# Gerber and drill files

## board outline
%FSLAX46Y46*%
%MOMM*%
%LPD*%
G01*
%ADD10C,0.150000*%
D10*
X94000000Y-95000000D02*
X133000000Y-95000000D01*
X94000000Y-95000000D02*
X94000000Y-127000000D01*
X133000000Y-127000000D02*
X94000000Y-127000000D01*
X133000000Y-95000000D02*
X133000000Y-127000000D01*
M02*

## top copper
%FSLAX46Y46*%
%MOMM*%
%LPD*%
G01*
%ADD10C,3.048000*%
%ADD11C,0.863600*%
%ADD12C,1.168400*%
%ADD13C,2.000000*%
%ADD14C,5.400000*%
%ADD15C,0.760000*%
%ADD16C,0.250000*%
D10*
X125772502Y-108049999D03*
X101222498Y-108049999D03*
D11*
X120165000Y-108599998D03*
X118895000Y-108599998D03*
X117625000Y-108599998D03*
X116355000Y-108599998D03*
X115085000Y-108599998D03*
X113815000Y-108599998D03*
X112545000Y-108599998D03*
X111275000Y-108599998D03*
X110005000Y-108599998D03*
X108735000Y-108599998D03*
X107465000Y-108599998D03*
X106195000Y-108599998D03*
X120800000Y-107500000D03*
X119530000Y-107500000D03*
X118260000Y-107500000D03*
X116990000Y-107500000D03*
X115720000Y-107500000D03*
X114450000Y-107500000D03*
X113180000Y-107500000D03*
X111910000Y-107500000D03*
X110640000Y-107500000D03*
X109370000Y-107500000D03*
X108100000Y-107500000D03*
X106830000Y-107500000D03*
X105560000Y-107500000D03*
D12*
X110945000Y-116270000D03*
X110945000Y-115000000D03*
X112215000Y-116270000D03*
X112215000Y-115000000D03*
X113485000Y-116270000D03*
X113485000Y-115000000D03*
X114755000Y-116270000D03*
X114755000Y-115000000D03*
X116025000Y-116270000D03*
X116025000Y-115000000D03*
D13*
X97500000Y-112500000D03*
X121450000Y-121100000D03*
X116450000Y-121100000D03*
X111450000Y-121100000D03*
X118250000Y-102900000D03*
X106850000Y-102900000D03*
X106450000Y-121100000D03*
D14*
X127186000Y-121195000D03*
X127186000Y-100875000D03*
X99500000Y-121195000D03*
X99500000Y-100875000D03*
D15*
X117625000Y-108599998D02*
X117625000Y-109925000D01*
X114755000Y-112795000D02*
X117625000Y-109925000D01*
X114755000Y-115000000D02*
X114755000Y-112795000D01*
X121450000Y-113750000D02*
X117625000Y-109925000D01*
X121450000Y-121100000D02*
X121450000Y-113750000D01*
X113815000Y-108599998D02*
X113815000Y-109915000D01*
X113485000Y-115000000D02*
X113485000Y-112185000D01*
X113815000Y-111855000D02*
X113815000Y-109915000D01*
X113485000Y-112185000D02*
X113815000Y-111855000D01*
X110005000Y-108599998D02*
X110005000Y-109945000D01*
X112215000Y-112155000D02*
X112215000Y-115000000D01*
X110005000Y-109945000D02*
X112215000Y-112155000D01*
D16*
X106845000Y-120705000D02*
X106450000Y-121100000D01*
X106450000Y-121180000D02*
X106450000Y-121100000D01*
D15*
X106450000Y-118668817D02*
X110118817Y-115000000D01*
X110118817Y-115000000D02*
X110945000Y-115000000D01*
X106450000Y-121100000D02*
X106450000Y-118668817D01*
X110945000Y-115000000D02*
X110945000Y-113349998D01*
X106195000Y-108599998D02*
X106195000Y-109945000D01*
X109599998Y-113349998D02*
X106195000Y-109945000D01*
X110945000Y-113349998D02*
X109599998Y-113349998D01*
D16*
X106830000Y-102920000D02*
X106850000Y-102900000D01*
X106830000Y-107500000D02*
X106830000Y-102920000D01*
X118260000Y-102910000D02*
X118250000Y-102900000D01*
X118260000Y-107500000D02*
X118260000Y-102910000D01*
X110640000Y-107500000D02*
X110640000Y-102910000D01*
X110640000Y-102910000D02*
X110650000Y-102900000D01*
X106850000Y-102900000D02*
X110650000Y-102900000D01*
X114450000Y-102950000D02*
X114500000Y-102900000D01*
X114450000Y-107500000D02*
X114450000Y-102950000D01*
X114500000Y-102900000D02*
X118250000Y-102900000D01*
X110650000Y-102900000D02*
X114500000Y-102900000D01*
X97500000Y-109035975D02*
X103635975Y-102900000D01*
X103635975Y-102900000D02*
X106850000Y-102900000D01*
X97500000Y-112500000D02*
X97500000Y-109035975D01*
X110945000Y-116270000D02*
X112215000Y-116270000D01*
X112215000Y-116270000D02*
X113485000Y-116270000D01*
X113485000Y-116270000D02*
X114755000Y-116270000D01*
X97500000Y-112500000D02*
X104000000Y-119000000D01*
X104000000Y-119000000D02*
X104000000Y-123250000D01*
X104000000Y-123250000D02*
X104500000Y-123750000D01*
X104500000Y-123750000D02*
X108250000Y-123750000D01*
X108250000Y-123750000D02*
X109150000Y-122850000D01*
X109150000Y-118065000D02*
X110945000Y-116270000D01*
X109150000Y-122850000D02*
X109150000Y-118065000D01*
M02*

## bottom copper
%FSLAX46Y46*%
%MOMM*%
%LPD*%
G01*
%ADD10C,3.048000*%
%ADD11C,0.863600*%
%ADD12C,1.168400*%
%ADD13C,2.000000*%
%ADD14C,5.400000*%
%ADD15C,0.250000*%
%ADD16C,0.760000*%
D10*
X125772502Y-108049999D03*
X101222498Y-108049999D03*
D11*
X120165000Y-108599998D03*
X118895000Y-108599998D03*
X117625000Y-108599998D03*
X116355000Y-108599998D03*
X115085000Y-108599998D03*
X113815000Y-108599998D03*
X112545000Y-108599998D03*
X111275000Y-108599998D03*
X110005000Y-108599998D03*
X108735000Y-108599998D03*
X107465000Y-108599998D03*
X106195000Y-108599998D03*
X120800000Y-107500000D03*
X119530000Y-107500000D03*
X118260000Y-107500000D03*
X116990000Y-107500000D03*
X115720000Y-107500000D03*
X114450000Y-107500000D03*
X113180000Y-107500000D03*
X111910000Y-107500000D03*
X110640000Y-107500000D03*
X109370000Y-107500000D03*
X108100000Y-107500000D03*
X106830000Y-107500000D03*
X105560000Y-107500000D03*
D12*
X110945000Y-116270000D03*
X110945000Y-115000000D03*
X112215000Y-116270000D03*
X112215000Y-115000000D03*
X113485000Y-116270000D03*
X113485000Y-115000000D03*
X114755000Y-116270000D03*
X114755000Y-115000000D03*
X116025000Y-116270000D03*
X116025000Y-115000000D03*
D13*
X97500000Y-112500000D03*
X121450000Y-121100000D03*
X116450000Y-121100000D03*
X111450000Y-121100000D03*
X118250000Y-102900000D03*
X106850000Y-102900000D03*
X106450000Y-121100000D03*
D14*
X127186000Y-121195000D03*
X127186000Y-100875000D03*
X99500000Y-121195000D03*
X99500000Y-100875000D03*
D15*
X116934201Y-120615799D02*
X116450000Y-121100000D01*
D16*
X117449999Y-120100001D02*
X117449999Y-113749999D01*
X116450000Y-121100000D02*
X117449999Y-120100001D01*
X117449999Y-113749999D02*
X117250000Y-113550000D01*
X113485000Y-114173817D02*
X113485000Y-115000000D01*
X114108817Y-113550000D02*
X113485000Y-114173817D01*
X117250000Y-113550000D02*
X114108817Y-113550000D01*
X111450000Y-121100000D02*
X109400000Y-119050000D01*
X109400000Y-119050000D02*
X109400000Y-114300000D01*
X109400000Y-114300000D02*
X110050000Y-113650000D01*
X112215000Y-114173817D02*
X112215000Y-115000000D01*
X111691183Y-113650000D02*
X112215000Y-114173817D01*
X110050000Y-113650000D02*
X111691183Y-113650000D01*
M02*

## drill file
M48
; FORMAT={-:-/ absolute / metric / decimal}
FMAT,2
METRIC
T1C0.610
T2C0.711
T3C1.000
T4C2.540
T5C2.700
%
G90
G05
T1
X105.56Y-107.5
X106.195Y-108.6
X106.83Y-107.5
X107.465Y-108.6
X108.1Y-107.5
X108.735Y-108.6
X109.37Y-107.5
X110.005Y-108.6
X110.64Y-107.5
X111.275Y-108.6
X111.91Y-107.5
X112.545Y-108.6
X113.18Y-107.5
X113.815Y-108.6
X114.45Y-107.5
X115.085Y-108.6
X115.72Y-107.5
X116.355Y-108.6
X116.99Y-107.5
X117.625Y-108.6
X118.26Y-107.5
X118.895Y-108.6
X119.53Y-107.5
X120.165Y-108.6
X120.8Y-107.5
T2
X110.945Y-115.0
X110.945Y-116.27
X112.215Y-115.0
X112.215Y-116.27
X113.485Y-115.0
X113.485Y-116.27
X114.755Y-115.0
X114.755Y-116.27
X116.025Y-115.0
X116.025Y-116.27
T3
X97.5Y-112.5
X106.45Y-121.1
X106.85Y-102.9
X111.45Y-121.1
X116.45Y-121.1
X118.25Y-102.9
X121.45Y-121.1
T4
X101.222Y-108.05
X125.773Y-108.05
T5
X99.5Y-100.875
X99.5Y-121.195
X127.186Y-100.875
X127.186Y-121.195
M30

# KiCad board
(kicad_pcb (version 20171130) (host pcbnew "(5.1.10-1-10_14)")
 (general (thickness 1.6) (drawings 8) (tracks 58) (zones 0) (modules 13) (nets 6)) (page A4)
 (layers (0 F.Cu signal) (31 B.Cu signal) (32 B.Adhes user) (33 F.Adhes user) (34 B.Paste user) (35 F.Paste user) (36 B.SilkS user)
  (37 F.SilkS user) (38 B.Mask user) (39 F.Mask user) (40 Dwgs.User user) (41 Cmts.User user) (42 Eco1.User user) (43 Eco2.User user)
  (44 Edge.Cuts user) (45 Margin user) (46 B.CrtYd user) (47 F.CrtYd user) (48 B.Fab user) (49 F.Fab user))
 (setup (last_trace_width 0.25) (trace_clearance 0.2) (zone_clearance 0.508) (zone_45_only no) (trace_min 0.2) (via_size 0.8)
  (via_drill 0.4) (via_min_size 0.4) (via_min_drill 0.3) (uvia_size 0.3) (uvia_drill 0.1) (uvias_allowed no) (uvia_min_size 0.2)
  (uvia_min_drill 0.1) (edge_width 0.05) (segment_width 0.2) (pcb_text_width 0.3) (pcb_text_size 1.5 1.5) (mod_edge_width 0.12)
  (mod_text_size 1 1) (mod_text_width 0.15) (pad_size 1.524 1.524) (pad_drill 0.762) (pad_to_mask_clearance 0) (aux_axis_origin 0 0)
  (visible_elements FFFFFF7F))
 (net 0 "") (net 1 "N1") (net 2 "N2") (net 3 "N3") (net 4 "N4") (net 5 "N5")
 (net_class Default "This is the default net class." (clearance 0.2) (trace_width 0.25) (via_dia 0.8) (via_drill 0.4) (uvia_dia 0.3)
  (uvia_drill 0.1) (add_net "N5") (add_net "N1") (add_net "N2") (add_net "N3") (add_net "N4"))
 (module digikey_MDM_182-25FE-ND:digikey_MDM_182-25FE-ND (layer F.Cu) (at 120.8 107.5)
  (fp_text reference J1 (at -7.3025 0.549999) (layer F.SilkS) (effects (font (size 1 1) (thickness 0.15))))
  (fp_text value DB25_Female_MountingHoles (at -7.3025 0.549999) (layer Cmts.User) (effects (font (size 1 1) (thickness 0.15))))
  (pad 28 thru_hole circle (at 4.972502 0.549999 90) (size 3.048 3.048) (drill 2.54) (layers *.Cu *.Mask))
  (pad 27 thru_hole circle (at -19.577502 0.549999 90) (size 3.048 3.048) (drill 2.54) (layers *.Cu *.Mask))
  (pad 14 thru_hole circle (at -0.635 1.099998) (size 0.8636 0.8636) (drill 0.6096) (layers *.Cu *.Mask))
  (pad 15 thru_hole circle (at -1.905 1.099998) (size 0.8636 0.8636) (drill 0.6096) (layers *.Cu *.Mask))
  (pad 16 thru_hole circle (at -3.175 1.099998) (size 0.8636 0.8636) (drill 0.6096) (layers *.Cu *.Mask) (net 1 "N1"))
  (pad 17 thru_hole circle (at -4.445 1.099998) (size 0.8636 0.8636) (drill 0.6096) (layers *.Cu *.Mask))
  (pad 18 thru_hole circle (at -5.715 1.099998) (size 0.8636 0.8636) (drill 0.6096) (layers *.Cu *.Mask))
  (pad 19 thru_hole circle (at -6.985 1.099998) (size 0.8636 0.8636) (drill 0.6096) (layers *.Cu *.Mask) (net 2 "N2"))
  (pad 20 thru_hole circle (at -8.255 1.099998) (size 0.8636 0.8636) (drill 0.6096) (layers *.Cu *.Mask))
  (pad 21 thru_hole circle (at -9.525 1.099998) (size 0.8636 0.8636) (drill 0.6096) (layers *.Cu *.Mask))
  (pad 22 thru_hole circle (at -10.795 1.099998) (size 0.8636 0.8636) (drill 0.6096) (layers *.Cu *.Mask) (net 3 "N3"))
  (pad 23 thru_hole circle (at -12.065 1.099998) (size 0.8636 0.8636) (drill 0.6096) (layers *.Cu *.Mask))
  (pad 24 thru_hole circle (at -13.335 1.099998) (size 0.8636 0.8636) (drill 0.6096) (layers *.Cu *.Mask))
  (pad 25 thru_hole circle (at -14.605 1.099998) (size 0.8636 0.8636) (drill 0.6096) (layers *.Cu *.Mask) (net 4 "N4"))
  (pad 1 thru_hole circle (at 0 0) (size 0.8636 0.8636) (drill 0.6096) (layers *.Cu *.Mask))
  (pad 2 thru_hole circle (at -1.27 0) (size 0.8636 0.8636) (drill 0.6096) (layers *.Cu *.Mask))
  (pad 3 thru_hole circle (at -2.54 0) (size 0.8636 0.8636) (drill 0.6096) (layers *.Cu *.Mask) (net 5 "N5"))
  (pad 4 thru_hole circle (at -3.81 0) (size 0.8636 0.8636) (drill 0.6096) (layers *.Cu *.Mask))
  (pad 5 thru_hole circle (at -5.08 0) (size 0.8636 0.8636) (drill 0.6096) (layers *.Cu *.Mask))
  (pad 6 thru_hole circle (at -6.35 0) (size 0.8636 0.8636) (drill 0.6096) (layers *.Cu *.Mask) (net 5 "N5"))
  (pad 7 thru_hole circle (at -7.62 0) (size 0.8636 0.8636) (drill 0.6096) (layers *.Cu *.Mask))
  (pad 8 thru_hole circle (at -8.89 0) (size 0.8636 0.8636) (drill 0.6096) (layers *.Cu *.Mask))
  (pad 9 thru_hole circle (at -10.16 0) (size 0.8636 0.8636) (drill 0.6096) (layers *.Cu *.Mask) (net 5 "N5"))
  (pad 10 thru_hole circle (at -11.43 0) (size 0.8636 0.8636) (drill 0.6096) (layers *.Cu *.Mask))
  (pad 11 thru_hole circle (at -12.7 0) (size 0.8636 0.8636) (drill 0.6096) (layers *.Cu *.Mask))
  (pad 12 thru_hole circle (at -13.97 0) (size 0.8636 0.8636) (drill 0.6096) (layers *.Cu *.Mask) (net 5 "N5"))
  (pad 13 thru_hole circle (at -15.24 0) (size 0.8636 0.8636) (drill 0.6096) (layers *.Cu *.Mask)))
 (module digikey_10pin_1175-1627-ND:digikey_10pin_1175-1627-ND (layer F.Cu) (at 116.025 115 180)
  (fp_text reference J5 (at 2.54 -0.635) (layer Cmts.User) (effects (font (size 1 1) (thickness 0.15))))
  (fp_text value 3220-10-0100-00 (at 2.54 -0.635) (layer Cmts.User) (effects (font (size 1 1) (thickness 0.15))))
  (pad 10 thru_hole circle (at 5.08 -1.27 180) (size 1.1684 1.1684) (drill 0.7112) (layers *.Cu *.Mask) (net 5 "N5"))
  (pad 9 thru_hole circle (at 5.08 0 180) (size 1.1684 1.1684) (drill 0.7112) (layers *.Cu *.Mask) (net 4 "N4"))
  (pad 8 thru_hole circle (at 3.81 -1.27 180) (size 1.1684 1.1684) (drill 0.7112) (layers *.Cu *.Mask) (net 5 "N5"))
  (pad 7 thru_hole circle (at 3.81 0 180) (size 1.1684 1.1684) (drill 0.7112) (layers *.Cu *.Mask) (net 3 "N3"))
  (pad 6 thru_hole circle (at 2.54 -1.27 180) (size 1.1684 1.1684) (drill 0.7112) (layers *.Cu *.Mask) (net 5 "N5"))
  (pad 5 thru_hole circle (at 2.54 0 180) (size 1.1684 1.1684) (drill 0.7112) (layers *.Cu *.Mask) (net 2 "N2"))
  (pad 4 thru_hole circle (at 1.27 -1.27 180) (size 1.1684 1.1684) (drill 0.7112) (layers *.Cu *.Mask) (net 5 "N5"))
  (pad 3 thru_hole circle (at 1.27 0 180) (size 1.1684 1.1684) (drill 0.7112) (layers *.Cu *.Mask) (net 1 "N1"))
  (pad 2 thru_hole circle (at 0 -1.27 180) (size 1.1684 1.1684) (drill 0.7112) (layers *.Cu *.Mask))
  (pad 1 thru_hole circle (at 0 0 180) (size 1.1684 1.1684) (drill 0.7112) (layers *.Cu *.Mask)))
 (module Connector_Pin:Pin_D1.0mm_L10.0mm (layer F.Cu) (at 97.5 112.5)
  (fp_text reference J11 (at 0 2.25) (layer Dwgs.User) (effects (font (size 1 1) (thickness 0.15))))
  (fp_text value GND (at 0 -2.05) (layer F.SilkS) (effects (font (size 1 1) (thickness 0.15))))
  (pad 1 thru_hole circle (at 0 0) (size 2 2) (drill 1) (layers *.Cu *.Mask) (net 5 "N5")))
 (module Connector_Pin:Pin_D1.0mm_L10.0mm (layer F.Cu) (at 121.45 121.1)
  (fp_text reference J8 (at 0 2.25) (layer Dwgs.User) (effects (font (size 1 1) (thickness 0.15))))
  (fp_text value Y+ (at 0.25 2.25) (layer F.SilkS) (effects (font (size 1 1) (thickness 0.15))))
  (pad 1 thru_hole circle (at 0 0) (size 2 2) (drill 1) (layers *.Cu *.Mask) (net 1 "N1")))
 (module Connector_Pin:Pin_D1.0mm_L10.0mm (layer F.Cu) (at 116.45 121.1)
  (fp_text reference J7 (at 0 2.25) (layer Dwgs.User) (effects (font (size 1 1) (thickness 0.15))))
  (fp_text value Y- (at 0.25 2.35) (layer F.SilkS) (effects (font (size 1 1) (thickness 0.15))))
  (pad 1 thru_hole circle (at 0 0) (size 2 2) (drill 1) (layers *.Cu *.Mask) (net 2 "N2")))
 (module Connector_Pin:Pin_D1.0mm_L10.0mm (layer F.Cu) (at 111.45 121.1)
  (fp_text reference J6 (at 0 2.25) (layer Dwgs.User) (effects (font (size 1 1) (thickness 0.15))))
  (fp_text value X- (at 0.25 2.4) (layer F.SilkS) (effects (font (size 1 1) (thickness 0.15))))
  (pad 1 thru_hole circle (at 0 0) (size 2 2) (drill 1) (layers *.Cu *.Mask) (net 3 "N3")))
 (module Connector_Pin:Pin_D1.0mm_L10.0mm (layer F.Cu) (at 118.25 102.9)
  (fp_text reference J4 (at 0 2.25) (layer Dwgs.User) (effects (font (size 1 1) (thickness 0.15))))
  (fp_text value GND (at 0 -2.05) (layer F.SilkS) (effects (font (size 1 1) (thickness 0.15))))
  (pad 1 thru_hole circle (at 0 0) (size 2 2) (drill 1) (layers *.Cu *.Mask) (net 5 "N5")))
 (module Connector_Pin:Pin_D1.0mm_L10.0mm (layer F.Cu) (at 106.85 102.9)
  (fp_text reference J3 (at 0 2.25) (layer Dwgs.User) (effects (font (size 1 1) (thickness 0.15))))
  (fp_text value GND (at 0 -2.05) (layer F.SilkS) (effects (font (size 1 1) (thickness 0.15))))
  (pad 1 thru_hole circle (at 0 0) (size 2 2) (drill 1) (layers *.Cu *.Mask) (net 5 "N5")))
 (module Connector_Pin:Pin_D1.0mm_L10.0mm (layer F.Cu) (at 106.45 121.1)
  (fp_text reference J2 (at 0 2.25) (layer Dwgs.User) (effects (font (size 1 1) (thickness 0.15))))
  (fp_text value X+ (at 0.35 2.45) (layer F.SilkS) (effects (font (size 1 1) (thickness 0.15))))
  (pad 1 thru_hole circle (at 0 0) (size 2 2) (drill 1) (layers *.Cu *.Mask) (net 4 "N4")))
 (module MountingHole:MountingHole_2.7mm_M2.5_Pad (layer F.Cu) (at 127.186 121.195)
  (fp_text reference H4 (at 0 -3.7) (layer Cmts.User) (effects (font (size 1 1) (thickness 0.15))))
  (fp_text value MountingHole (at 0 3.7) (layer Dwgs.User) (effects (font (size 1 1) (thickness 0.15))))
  (pad 1 thru_hole circle (at 0 0) (size 5.4 5.4) (drill 2.7) (layers *.Cu *.Mask)))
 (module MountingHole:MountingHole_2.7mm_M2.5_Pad (layer F.Cu) (at 127.186 100.875)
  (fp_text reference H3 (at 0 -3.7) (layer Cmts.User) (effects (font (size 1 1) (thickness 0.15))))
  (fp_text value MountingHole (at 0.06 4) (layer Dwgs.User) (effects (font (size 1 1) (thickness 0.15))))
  (pad 1 thru_hole circle (at 0 0) (size 5.4 5.4) (drill 2.7) (layers *.Cu *.Mask)))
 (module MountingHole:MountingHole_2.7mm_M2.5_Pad (layer F.Cu) (at 99.5 121.195)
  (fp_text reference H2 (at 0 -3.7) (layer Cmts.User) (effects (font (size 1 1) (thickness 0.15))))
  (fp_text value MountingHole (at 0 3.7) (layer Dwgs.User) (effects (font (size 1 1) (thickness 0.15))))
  (pad 1 thru_hole circle (at 0 0) (size 5.4 5.4) (drill 2.7) (layers *.Cu *.Mask)))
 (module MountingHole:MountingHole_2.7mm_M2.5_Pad (layer F.Cu) (at 99.5 100.875)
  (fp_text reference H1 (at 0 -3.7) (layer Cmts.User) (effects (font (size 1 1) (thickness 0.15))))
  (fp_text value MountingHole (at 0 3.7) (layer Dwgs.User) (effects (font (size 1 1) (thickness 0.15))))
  (pad 1 thru_hole circle (at 0 0) (size 5.4 5.4) (drill 2.7) (layers *.Cu *.Mask)))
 (gr_line (start 94 95) (end 133 95) (layer Edge.Cuts) (width 0.15))
 (gr_line (start 94 95) (end 94 127) (layer Edge.Cuts) (width 0.15))
 (gr_line (start 133 127) (end 94 127) (layer Edge.Cuts) (width 0.15))
 (gr_line (start 133 95) (end 133 127) (layer Edge.Cuts) (width 0.15))
 (segment (start 117.625 108.599998) (end 117.625 109.925) (width 0.76) (layer F.Cu) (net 1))
 (segment (start 114.755 112.795) (end 117.625 109.925) (width 0.76) (layer F.Cu) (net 1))
 (segment (start 114.755 115) (end 114.755 112.795) (width 0.76) (layer F.Cu) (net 1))
 (segment (start 121.45 113.75) (end 117.625 109.925) (width 0.76) (layer F.Cu) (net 1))
 (segment (start 121.45 121.1) (end 121.45 113.75) (width 0.76) (layer F.Cu) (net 1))
 (segment (start 116.934201 120.615799) (end 116.45 121.1) (width 0.25) (layer B.Cu) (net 2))
 (segment (start 117.449999 120.100001) (end 117.449999 113.749999) (width 0.76) (layer B.Cu) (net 2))
 (segment (start 116.45 121.1) (end 117.449999 120.100001) (width 0.76) (layer B.Cu) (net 2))
 (segment (start 117.449999 113.749999) (end 117.25 113.55) (width 0.76) (layer B.Cu) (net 2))
 (segment (start 113.485 114.173817) (end 113.485 115) (width 0.76) (layer B.Cu) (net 2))
 (segment (start 114.108817 113.55) (end 113.485 114.173817) (width 0.76) (layer B.Cu) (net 2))
 (segment (start 117.25 113.55) (end 114.108817 113.55) (width 0.76) (layer B.Cu) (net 2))
 (segment (start 113.815 108.599998) (end 113.815 109.915) (width 0.76) (layer F.Cu) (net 2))
 (segment (start 113.485 115) (end 113.485 112.185) (width 0.76) (layer F.Cu) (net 2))
 (segment (start 113.815 111.855) (end 113.815 109.915) (width 0.76) (layer F.Cu) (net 2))
 (segment (start 113.485 112.185) (end 113.815 111.855) (width 0.76) (layer F.Cu) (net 2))
 (segment (start 111.45 121.1) (end 109.4 119.05) (width 0.76) (layer B.Cu) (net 3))
 (segment (start 109.4 119.05) (end 109.4 114.3) (width 0.76) (layer B.Cu) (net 3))
 (segment (start 109.4 114.3) (end 110.05 113.65) (width 0.76) (layer B.Cu) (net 3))
 (segment (start 112.215 114.173817) (end 112.215 115) (width 0.76) (layer B.Cu) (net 3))
 (segment (start 111.691183 113.65) (end 112.215 114.173817) (width 0.76) (layer B.Cu) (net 3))
 (segment (start 110.05 113.65) (end 111.691183 113.65) (width 0.76) (layer B.Cu) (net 3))
 (segment (start 110.005 108.599998) (end 110.005 109.945) (width 0.76) (layer F.Cu) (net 3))
 (segment (start 112.215 112.155) (end 112.215 115) (width 0.76) (layer F.Cu) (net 3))
 (segment (start 110.005 109.945) (end 112.215 112.155) (width 0.76) (layer F.Cu) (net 3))
 (segment (start 106.845 120.705) (end 106.45 121.1) (width 0.25) (layer F.Cu) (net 4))
 (segment (start 106.45 121.18) (end 106.45 121.1) (width 0.25) (layer F.Cu) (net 4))
 (segment (start 106.45 118.668817) (end 110.118817 115) (width 0.76) (layer F.Cu) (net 4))
 (segment (start 110.118817 115) (end 110.945 115) (width 0.76) (layer F.Cu) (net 4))
 (segment (start 106.45 121.1) (end 106.45 118.668817) (width 0.76) (layer F.Cu) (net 4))
 (segment (start 110.945 115) (end 110.945 113.349998) (width 0.76) (layer F.Cu) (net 4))
 (segment (start 106.195 108.599998) (end 106.195 109.945) (width 0.76) (layer F.Cu) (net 4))
 (segment (start 109.599998 113.349998) (end 106.195 109.945) (width 0.76) (layer F.Cu) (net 4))
 (segment (start 110.945 113.349998) (end 109.599998 113.349998) (width 0.76) (layer F.Cu) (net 4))
 (segment (start 106.83 102.92) (end 106.85 102.9) (width 0.25) (layer F.Cu) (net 5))
 (segment (start 106.83 107.5) (end 106.83 102.92) (width 0.25) (layer F.Cu) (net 5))
 (segment (start 118.26 102.91) (end 118.25 102.9) (width 0.25) (layer F.Cu) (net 5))
 (segment (start 118.26 107.5) (end 118.26 102.91) (width 0.25) (layer F.Cu) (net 5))
 (segment (start 110.64 107.5) (end 110.64 102.91) (width 0.25) (layer F.Cu) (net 5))
 (segment (start 110.64 102.91) (end 110.65 102.9) (width 0.25) (layer F.Cu) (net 5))
 (segment (start 106.85 102.9) (end 110.65 102.9) (width 0.25) (layer F.Cu) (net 5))
 (segment (start 114.45 102.95) (end 114.5 102.9) (width 0.25) (layer F.Cu) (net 5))
 (segment (start 114.45 107.5) (end 114.45 102.95) (width 0.25) (layer F.Cu) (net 5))
 (segment (start 114.5 102.9) (end 118.25 102.9) (width 0.25) (layer F.Cu) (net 5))
 (segment (start 110.65 102.9) (end 114.5 102.9) (width 0.25) (layer F.Cu) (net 5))
 (segment (start 97.5 109.035975) (end 103.635975 102.9) (width 0.25) (layer F.Cu) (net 5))
 (segment (start 103.635975 102.9) (end 106.85 102.9) (width 0.25) (layer F.Cu) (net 5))
 (segment (start 97.5 112.5) (end 97.5 109.035975) (width 0.25) (layer F.Cu) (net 5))
 (segment (start 110.945 116.27) (end 112.215 116.27) (width 0.25) (layer F.Cu) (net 5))
 (segment (start 112.215 116.27) (end 113.485 116.27) (width 0.25) (layer F.Cu) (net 5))
 (segment (start 113.485 116.27) (end 114.755 116.27) (width 0.25) (layer F.Cu) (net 5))
 (segment (start 97.5 112.5) (end 104 119) (width 0.25) (layer F.Cu) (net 5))
 (segment (start 104 119) (end 104 123.25) (width 0.25) (layer F.Cu) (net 5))
 (segment (start 104 123.25) (end 104.5 123.75) (width 0.25) (layer F.Cu) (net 5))
 (segment (start 104.5 123.75) (end 108.25 123.75) (width 0.25) (layer F.Cu) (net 5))
 (segment (start 108.25 123.75) (end 109.15 122.85) (width 0.25) (layer F.Cu) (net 5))
 (segment (start 109.15 118.065) (end 110.945 116.27) (width 0.25) (layer F.Cu) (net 5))
 (segment (start 109.15 122.85) (end 109.15 118.065) (width 0.25) (layer F.Cu) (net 5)))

